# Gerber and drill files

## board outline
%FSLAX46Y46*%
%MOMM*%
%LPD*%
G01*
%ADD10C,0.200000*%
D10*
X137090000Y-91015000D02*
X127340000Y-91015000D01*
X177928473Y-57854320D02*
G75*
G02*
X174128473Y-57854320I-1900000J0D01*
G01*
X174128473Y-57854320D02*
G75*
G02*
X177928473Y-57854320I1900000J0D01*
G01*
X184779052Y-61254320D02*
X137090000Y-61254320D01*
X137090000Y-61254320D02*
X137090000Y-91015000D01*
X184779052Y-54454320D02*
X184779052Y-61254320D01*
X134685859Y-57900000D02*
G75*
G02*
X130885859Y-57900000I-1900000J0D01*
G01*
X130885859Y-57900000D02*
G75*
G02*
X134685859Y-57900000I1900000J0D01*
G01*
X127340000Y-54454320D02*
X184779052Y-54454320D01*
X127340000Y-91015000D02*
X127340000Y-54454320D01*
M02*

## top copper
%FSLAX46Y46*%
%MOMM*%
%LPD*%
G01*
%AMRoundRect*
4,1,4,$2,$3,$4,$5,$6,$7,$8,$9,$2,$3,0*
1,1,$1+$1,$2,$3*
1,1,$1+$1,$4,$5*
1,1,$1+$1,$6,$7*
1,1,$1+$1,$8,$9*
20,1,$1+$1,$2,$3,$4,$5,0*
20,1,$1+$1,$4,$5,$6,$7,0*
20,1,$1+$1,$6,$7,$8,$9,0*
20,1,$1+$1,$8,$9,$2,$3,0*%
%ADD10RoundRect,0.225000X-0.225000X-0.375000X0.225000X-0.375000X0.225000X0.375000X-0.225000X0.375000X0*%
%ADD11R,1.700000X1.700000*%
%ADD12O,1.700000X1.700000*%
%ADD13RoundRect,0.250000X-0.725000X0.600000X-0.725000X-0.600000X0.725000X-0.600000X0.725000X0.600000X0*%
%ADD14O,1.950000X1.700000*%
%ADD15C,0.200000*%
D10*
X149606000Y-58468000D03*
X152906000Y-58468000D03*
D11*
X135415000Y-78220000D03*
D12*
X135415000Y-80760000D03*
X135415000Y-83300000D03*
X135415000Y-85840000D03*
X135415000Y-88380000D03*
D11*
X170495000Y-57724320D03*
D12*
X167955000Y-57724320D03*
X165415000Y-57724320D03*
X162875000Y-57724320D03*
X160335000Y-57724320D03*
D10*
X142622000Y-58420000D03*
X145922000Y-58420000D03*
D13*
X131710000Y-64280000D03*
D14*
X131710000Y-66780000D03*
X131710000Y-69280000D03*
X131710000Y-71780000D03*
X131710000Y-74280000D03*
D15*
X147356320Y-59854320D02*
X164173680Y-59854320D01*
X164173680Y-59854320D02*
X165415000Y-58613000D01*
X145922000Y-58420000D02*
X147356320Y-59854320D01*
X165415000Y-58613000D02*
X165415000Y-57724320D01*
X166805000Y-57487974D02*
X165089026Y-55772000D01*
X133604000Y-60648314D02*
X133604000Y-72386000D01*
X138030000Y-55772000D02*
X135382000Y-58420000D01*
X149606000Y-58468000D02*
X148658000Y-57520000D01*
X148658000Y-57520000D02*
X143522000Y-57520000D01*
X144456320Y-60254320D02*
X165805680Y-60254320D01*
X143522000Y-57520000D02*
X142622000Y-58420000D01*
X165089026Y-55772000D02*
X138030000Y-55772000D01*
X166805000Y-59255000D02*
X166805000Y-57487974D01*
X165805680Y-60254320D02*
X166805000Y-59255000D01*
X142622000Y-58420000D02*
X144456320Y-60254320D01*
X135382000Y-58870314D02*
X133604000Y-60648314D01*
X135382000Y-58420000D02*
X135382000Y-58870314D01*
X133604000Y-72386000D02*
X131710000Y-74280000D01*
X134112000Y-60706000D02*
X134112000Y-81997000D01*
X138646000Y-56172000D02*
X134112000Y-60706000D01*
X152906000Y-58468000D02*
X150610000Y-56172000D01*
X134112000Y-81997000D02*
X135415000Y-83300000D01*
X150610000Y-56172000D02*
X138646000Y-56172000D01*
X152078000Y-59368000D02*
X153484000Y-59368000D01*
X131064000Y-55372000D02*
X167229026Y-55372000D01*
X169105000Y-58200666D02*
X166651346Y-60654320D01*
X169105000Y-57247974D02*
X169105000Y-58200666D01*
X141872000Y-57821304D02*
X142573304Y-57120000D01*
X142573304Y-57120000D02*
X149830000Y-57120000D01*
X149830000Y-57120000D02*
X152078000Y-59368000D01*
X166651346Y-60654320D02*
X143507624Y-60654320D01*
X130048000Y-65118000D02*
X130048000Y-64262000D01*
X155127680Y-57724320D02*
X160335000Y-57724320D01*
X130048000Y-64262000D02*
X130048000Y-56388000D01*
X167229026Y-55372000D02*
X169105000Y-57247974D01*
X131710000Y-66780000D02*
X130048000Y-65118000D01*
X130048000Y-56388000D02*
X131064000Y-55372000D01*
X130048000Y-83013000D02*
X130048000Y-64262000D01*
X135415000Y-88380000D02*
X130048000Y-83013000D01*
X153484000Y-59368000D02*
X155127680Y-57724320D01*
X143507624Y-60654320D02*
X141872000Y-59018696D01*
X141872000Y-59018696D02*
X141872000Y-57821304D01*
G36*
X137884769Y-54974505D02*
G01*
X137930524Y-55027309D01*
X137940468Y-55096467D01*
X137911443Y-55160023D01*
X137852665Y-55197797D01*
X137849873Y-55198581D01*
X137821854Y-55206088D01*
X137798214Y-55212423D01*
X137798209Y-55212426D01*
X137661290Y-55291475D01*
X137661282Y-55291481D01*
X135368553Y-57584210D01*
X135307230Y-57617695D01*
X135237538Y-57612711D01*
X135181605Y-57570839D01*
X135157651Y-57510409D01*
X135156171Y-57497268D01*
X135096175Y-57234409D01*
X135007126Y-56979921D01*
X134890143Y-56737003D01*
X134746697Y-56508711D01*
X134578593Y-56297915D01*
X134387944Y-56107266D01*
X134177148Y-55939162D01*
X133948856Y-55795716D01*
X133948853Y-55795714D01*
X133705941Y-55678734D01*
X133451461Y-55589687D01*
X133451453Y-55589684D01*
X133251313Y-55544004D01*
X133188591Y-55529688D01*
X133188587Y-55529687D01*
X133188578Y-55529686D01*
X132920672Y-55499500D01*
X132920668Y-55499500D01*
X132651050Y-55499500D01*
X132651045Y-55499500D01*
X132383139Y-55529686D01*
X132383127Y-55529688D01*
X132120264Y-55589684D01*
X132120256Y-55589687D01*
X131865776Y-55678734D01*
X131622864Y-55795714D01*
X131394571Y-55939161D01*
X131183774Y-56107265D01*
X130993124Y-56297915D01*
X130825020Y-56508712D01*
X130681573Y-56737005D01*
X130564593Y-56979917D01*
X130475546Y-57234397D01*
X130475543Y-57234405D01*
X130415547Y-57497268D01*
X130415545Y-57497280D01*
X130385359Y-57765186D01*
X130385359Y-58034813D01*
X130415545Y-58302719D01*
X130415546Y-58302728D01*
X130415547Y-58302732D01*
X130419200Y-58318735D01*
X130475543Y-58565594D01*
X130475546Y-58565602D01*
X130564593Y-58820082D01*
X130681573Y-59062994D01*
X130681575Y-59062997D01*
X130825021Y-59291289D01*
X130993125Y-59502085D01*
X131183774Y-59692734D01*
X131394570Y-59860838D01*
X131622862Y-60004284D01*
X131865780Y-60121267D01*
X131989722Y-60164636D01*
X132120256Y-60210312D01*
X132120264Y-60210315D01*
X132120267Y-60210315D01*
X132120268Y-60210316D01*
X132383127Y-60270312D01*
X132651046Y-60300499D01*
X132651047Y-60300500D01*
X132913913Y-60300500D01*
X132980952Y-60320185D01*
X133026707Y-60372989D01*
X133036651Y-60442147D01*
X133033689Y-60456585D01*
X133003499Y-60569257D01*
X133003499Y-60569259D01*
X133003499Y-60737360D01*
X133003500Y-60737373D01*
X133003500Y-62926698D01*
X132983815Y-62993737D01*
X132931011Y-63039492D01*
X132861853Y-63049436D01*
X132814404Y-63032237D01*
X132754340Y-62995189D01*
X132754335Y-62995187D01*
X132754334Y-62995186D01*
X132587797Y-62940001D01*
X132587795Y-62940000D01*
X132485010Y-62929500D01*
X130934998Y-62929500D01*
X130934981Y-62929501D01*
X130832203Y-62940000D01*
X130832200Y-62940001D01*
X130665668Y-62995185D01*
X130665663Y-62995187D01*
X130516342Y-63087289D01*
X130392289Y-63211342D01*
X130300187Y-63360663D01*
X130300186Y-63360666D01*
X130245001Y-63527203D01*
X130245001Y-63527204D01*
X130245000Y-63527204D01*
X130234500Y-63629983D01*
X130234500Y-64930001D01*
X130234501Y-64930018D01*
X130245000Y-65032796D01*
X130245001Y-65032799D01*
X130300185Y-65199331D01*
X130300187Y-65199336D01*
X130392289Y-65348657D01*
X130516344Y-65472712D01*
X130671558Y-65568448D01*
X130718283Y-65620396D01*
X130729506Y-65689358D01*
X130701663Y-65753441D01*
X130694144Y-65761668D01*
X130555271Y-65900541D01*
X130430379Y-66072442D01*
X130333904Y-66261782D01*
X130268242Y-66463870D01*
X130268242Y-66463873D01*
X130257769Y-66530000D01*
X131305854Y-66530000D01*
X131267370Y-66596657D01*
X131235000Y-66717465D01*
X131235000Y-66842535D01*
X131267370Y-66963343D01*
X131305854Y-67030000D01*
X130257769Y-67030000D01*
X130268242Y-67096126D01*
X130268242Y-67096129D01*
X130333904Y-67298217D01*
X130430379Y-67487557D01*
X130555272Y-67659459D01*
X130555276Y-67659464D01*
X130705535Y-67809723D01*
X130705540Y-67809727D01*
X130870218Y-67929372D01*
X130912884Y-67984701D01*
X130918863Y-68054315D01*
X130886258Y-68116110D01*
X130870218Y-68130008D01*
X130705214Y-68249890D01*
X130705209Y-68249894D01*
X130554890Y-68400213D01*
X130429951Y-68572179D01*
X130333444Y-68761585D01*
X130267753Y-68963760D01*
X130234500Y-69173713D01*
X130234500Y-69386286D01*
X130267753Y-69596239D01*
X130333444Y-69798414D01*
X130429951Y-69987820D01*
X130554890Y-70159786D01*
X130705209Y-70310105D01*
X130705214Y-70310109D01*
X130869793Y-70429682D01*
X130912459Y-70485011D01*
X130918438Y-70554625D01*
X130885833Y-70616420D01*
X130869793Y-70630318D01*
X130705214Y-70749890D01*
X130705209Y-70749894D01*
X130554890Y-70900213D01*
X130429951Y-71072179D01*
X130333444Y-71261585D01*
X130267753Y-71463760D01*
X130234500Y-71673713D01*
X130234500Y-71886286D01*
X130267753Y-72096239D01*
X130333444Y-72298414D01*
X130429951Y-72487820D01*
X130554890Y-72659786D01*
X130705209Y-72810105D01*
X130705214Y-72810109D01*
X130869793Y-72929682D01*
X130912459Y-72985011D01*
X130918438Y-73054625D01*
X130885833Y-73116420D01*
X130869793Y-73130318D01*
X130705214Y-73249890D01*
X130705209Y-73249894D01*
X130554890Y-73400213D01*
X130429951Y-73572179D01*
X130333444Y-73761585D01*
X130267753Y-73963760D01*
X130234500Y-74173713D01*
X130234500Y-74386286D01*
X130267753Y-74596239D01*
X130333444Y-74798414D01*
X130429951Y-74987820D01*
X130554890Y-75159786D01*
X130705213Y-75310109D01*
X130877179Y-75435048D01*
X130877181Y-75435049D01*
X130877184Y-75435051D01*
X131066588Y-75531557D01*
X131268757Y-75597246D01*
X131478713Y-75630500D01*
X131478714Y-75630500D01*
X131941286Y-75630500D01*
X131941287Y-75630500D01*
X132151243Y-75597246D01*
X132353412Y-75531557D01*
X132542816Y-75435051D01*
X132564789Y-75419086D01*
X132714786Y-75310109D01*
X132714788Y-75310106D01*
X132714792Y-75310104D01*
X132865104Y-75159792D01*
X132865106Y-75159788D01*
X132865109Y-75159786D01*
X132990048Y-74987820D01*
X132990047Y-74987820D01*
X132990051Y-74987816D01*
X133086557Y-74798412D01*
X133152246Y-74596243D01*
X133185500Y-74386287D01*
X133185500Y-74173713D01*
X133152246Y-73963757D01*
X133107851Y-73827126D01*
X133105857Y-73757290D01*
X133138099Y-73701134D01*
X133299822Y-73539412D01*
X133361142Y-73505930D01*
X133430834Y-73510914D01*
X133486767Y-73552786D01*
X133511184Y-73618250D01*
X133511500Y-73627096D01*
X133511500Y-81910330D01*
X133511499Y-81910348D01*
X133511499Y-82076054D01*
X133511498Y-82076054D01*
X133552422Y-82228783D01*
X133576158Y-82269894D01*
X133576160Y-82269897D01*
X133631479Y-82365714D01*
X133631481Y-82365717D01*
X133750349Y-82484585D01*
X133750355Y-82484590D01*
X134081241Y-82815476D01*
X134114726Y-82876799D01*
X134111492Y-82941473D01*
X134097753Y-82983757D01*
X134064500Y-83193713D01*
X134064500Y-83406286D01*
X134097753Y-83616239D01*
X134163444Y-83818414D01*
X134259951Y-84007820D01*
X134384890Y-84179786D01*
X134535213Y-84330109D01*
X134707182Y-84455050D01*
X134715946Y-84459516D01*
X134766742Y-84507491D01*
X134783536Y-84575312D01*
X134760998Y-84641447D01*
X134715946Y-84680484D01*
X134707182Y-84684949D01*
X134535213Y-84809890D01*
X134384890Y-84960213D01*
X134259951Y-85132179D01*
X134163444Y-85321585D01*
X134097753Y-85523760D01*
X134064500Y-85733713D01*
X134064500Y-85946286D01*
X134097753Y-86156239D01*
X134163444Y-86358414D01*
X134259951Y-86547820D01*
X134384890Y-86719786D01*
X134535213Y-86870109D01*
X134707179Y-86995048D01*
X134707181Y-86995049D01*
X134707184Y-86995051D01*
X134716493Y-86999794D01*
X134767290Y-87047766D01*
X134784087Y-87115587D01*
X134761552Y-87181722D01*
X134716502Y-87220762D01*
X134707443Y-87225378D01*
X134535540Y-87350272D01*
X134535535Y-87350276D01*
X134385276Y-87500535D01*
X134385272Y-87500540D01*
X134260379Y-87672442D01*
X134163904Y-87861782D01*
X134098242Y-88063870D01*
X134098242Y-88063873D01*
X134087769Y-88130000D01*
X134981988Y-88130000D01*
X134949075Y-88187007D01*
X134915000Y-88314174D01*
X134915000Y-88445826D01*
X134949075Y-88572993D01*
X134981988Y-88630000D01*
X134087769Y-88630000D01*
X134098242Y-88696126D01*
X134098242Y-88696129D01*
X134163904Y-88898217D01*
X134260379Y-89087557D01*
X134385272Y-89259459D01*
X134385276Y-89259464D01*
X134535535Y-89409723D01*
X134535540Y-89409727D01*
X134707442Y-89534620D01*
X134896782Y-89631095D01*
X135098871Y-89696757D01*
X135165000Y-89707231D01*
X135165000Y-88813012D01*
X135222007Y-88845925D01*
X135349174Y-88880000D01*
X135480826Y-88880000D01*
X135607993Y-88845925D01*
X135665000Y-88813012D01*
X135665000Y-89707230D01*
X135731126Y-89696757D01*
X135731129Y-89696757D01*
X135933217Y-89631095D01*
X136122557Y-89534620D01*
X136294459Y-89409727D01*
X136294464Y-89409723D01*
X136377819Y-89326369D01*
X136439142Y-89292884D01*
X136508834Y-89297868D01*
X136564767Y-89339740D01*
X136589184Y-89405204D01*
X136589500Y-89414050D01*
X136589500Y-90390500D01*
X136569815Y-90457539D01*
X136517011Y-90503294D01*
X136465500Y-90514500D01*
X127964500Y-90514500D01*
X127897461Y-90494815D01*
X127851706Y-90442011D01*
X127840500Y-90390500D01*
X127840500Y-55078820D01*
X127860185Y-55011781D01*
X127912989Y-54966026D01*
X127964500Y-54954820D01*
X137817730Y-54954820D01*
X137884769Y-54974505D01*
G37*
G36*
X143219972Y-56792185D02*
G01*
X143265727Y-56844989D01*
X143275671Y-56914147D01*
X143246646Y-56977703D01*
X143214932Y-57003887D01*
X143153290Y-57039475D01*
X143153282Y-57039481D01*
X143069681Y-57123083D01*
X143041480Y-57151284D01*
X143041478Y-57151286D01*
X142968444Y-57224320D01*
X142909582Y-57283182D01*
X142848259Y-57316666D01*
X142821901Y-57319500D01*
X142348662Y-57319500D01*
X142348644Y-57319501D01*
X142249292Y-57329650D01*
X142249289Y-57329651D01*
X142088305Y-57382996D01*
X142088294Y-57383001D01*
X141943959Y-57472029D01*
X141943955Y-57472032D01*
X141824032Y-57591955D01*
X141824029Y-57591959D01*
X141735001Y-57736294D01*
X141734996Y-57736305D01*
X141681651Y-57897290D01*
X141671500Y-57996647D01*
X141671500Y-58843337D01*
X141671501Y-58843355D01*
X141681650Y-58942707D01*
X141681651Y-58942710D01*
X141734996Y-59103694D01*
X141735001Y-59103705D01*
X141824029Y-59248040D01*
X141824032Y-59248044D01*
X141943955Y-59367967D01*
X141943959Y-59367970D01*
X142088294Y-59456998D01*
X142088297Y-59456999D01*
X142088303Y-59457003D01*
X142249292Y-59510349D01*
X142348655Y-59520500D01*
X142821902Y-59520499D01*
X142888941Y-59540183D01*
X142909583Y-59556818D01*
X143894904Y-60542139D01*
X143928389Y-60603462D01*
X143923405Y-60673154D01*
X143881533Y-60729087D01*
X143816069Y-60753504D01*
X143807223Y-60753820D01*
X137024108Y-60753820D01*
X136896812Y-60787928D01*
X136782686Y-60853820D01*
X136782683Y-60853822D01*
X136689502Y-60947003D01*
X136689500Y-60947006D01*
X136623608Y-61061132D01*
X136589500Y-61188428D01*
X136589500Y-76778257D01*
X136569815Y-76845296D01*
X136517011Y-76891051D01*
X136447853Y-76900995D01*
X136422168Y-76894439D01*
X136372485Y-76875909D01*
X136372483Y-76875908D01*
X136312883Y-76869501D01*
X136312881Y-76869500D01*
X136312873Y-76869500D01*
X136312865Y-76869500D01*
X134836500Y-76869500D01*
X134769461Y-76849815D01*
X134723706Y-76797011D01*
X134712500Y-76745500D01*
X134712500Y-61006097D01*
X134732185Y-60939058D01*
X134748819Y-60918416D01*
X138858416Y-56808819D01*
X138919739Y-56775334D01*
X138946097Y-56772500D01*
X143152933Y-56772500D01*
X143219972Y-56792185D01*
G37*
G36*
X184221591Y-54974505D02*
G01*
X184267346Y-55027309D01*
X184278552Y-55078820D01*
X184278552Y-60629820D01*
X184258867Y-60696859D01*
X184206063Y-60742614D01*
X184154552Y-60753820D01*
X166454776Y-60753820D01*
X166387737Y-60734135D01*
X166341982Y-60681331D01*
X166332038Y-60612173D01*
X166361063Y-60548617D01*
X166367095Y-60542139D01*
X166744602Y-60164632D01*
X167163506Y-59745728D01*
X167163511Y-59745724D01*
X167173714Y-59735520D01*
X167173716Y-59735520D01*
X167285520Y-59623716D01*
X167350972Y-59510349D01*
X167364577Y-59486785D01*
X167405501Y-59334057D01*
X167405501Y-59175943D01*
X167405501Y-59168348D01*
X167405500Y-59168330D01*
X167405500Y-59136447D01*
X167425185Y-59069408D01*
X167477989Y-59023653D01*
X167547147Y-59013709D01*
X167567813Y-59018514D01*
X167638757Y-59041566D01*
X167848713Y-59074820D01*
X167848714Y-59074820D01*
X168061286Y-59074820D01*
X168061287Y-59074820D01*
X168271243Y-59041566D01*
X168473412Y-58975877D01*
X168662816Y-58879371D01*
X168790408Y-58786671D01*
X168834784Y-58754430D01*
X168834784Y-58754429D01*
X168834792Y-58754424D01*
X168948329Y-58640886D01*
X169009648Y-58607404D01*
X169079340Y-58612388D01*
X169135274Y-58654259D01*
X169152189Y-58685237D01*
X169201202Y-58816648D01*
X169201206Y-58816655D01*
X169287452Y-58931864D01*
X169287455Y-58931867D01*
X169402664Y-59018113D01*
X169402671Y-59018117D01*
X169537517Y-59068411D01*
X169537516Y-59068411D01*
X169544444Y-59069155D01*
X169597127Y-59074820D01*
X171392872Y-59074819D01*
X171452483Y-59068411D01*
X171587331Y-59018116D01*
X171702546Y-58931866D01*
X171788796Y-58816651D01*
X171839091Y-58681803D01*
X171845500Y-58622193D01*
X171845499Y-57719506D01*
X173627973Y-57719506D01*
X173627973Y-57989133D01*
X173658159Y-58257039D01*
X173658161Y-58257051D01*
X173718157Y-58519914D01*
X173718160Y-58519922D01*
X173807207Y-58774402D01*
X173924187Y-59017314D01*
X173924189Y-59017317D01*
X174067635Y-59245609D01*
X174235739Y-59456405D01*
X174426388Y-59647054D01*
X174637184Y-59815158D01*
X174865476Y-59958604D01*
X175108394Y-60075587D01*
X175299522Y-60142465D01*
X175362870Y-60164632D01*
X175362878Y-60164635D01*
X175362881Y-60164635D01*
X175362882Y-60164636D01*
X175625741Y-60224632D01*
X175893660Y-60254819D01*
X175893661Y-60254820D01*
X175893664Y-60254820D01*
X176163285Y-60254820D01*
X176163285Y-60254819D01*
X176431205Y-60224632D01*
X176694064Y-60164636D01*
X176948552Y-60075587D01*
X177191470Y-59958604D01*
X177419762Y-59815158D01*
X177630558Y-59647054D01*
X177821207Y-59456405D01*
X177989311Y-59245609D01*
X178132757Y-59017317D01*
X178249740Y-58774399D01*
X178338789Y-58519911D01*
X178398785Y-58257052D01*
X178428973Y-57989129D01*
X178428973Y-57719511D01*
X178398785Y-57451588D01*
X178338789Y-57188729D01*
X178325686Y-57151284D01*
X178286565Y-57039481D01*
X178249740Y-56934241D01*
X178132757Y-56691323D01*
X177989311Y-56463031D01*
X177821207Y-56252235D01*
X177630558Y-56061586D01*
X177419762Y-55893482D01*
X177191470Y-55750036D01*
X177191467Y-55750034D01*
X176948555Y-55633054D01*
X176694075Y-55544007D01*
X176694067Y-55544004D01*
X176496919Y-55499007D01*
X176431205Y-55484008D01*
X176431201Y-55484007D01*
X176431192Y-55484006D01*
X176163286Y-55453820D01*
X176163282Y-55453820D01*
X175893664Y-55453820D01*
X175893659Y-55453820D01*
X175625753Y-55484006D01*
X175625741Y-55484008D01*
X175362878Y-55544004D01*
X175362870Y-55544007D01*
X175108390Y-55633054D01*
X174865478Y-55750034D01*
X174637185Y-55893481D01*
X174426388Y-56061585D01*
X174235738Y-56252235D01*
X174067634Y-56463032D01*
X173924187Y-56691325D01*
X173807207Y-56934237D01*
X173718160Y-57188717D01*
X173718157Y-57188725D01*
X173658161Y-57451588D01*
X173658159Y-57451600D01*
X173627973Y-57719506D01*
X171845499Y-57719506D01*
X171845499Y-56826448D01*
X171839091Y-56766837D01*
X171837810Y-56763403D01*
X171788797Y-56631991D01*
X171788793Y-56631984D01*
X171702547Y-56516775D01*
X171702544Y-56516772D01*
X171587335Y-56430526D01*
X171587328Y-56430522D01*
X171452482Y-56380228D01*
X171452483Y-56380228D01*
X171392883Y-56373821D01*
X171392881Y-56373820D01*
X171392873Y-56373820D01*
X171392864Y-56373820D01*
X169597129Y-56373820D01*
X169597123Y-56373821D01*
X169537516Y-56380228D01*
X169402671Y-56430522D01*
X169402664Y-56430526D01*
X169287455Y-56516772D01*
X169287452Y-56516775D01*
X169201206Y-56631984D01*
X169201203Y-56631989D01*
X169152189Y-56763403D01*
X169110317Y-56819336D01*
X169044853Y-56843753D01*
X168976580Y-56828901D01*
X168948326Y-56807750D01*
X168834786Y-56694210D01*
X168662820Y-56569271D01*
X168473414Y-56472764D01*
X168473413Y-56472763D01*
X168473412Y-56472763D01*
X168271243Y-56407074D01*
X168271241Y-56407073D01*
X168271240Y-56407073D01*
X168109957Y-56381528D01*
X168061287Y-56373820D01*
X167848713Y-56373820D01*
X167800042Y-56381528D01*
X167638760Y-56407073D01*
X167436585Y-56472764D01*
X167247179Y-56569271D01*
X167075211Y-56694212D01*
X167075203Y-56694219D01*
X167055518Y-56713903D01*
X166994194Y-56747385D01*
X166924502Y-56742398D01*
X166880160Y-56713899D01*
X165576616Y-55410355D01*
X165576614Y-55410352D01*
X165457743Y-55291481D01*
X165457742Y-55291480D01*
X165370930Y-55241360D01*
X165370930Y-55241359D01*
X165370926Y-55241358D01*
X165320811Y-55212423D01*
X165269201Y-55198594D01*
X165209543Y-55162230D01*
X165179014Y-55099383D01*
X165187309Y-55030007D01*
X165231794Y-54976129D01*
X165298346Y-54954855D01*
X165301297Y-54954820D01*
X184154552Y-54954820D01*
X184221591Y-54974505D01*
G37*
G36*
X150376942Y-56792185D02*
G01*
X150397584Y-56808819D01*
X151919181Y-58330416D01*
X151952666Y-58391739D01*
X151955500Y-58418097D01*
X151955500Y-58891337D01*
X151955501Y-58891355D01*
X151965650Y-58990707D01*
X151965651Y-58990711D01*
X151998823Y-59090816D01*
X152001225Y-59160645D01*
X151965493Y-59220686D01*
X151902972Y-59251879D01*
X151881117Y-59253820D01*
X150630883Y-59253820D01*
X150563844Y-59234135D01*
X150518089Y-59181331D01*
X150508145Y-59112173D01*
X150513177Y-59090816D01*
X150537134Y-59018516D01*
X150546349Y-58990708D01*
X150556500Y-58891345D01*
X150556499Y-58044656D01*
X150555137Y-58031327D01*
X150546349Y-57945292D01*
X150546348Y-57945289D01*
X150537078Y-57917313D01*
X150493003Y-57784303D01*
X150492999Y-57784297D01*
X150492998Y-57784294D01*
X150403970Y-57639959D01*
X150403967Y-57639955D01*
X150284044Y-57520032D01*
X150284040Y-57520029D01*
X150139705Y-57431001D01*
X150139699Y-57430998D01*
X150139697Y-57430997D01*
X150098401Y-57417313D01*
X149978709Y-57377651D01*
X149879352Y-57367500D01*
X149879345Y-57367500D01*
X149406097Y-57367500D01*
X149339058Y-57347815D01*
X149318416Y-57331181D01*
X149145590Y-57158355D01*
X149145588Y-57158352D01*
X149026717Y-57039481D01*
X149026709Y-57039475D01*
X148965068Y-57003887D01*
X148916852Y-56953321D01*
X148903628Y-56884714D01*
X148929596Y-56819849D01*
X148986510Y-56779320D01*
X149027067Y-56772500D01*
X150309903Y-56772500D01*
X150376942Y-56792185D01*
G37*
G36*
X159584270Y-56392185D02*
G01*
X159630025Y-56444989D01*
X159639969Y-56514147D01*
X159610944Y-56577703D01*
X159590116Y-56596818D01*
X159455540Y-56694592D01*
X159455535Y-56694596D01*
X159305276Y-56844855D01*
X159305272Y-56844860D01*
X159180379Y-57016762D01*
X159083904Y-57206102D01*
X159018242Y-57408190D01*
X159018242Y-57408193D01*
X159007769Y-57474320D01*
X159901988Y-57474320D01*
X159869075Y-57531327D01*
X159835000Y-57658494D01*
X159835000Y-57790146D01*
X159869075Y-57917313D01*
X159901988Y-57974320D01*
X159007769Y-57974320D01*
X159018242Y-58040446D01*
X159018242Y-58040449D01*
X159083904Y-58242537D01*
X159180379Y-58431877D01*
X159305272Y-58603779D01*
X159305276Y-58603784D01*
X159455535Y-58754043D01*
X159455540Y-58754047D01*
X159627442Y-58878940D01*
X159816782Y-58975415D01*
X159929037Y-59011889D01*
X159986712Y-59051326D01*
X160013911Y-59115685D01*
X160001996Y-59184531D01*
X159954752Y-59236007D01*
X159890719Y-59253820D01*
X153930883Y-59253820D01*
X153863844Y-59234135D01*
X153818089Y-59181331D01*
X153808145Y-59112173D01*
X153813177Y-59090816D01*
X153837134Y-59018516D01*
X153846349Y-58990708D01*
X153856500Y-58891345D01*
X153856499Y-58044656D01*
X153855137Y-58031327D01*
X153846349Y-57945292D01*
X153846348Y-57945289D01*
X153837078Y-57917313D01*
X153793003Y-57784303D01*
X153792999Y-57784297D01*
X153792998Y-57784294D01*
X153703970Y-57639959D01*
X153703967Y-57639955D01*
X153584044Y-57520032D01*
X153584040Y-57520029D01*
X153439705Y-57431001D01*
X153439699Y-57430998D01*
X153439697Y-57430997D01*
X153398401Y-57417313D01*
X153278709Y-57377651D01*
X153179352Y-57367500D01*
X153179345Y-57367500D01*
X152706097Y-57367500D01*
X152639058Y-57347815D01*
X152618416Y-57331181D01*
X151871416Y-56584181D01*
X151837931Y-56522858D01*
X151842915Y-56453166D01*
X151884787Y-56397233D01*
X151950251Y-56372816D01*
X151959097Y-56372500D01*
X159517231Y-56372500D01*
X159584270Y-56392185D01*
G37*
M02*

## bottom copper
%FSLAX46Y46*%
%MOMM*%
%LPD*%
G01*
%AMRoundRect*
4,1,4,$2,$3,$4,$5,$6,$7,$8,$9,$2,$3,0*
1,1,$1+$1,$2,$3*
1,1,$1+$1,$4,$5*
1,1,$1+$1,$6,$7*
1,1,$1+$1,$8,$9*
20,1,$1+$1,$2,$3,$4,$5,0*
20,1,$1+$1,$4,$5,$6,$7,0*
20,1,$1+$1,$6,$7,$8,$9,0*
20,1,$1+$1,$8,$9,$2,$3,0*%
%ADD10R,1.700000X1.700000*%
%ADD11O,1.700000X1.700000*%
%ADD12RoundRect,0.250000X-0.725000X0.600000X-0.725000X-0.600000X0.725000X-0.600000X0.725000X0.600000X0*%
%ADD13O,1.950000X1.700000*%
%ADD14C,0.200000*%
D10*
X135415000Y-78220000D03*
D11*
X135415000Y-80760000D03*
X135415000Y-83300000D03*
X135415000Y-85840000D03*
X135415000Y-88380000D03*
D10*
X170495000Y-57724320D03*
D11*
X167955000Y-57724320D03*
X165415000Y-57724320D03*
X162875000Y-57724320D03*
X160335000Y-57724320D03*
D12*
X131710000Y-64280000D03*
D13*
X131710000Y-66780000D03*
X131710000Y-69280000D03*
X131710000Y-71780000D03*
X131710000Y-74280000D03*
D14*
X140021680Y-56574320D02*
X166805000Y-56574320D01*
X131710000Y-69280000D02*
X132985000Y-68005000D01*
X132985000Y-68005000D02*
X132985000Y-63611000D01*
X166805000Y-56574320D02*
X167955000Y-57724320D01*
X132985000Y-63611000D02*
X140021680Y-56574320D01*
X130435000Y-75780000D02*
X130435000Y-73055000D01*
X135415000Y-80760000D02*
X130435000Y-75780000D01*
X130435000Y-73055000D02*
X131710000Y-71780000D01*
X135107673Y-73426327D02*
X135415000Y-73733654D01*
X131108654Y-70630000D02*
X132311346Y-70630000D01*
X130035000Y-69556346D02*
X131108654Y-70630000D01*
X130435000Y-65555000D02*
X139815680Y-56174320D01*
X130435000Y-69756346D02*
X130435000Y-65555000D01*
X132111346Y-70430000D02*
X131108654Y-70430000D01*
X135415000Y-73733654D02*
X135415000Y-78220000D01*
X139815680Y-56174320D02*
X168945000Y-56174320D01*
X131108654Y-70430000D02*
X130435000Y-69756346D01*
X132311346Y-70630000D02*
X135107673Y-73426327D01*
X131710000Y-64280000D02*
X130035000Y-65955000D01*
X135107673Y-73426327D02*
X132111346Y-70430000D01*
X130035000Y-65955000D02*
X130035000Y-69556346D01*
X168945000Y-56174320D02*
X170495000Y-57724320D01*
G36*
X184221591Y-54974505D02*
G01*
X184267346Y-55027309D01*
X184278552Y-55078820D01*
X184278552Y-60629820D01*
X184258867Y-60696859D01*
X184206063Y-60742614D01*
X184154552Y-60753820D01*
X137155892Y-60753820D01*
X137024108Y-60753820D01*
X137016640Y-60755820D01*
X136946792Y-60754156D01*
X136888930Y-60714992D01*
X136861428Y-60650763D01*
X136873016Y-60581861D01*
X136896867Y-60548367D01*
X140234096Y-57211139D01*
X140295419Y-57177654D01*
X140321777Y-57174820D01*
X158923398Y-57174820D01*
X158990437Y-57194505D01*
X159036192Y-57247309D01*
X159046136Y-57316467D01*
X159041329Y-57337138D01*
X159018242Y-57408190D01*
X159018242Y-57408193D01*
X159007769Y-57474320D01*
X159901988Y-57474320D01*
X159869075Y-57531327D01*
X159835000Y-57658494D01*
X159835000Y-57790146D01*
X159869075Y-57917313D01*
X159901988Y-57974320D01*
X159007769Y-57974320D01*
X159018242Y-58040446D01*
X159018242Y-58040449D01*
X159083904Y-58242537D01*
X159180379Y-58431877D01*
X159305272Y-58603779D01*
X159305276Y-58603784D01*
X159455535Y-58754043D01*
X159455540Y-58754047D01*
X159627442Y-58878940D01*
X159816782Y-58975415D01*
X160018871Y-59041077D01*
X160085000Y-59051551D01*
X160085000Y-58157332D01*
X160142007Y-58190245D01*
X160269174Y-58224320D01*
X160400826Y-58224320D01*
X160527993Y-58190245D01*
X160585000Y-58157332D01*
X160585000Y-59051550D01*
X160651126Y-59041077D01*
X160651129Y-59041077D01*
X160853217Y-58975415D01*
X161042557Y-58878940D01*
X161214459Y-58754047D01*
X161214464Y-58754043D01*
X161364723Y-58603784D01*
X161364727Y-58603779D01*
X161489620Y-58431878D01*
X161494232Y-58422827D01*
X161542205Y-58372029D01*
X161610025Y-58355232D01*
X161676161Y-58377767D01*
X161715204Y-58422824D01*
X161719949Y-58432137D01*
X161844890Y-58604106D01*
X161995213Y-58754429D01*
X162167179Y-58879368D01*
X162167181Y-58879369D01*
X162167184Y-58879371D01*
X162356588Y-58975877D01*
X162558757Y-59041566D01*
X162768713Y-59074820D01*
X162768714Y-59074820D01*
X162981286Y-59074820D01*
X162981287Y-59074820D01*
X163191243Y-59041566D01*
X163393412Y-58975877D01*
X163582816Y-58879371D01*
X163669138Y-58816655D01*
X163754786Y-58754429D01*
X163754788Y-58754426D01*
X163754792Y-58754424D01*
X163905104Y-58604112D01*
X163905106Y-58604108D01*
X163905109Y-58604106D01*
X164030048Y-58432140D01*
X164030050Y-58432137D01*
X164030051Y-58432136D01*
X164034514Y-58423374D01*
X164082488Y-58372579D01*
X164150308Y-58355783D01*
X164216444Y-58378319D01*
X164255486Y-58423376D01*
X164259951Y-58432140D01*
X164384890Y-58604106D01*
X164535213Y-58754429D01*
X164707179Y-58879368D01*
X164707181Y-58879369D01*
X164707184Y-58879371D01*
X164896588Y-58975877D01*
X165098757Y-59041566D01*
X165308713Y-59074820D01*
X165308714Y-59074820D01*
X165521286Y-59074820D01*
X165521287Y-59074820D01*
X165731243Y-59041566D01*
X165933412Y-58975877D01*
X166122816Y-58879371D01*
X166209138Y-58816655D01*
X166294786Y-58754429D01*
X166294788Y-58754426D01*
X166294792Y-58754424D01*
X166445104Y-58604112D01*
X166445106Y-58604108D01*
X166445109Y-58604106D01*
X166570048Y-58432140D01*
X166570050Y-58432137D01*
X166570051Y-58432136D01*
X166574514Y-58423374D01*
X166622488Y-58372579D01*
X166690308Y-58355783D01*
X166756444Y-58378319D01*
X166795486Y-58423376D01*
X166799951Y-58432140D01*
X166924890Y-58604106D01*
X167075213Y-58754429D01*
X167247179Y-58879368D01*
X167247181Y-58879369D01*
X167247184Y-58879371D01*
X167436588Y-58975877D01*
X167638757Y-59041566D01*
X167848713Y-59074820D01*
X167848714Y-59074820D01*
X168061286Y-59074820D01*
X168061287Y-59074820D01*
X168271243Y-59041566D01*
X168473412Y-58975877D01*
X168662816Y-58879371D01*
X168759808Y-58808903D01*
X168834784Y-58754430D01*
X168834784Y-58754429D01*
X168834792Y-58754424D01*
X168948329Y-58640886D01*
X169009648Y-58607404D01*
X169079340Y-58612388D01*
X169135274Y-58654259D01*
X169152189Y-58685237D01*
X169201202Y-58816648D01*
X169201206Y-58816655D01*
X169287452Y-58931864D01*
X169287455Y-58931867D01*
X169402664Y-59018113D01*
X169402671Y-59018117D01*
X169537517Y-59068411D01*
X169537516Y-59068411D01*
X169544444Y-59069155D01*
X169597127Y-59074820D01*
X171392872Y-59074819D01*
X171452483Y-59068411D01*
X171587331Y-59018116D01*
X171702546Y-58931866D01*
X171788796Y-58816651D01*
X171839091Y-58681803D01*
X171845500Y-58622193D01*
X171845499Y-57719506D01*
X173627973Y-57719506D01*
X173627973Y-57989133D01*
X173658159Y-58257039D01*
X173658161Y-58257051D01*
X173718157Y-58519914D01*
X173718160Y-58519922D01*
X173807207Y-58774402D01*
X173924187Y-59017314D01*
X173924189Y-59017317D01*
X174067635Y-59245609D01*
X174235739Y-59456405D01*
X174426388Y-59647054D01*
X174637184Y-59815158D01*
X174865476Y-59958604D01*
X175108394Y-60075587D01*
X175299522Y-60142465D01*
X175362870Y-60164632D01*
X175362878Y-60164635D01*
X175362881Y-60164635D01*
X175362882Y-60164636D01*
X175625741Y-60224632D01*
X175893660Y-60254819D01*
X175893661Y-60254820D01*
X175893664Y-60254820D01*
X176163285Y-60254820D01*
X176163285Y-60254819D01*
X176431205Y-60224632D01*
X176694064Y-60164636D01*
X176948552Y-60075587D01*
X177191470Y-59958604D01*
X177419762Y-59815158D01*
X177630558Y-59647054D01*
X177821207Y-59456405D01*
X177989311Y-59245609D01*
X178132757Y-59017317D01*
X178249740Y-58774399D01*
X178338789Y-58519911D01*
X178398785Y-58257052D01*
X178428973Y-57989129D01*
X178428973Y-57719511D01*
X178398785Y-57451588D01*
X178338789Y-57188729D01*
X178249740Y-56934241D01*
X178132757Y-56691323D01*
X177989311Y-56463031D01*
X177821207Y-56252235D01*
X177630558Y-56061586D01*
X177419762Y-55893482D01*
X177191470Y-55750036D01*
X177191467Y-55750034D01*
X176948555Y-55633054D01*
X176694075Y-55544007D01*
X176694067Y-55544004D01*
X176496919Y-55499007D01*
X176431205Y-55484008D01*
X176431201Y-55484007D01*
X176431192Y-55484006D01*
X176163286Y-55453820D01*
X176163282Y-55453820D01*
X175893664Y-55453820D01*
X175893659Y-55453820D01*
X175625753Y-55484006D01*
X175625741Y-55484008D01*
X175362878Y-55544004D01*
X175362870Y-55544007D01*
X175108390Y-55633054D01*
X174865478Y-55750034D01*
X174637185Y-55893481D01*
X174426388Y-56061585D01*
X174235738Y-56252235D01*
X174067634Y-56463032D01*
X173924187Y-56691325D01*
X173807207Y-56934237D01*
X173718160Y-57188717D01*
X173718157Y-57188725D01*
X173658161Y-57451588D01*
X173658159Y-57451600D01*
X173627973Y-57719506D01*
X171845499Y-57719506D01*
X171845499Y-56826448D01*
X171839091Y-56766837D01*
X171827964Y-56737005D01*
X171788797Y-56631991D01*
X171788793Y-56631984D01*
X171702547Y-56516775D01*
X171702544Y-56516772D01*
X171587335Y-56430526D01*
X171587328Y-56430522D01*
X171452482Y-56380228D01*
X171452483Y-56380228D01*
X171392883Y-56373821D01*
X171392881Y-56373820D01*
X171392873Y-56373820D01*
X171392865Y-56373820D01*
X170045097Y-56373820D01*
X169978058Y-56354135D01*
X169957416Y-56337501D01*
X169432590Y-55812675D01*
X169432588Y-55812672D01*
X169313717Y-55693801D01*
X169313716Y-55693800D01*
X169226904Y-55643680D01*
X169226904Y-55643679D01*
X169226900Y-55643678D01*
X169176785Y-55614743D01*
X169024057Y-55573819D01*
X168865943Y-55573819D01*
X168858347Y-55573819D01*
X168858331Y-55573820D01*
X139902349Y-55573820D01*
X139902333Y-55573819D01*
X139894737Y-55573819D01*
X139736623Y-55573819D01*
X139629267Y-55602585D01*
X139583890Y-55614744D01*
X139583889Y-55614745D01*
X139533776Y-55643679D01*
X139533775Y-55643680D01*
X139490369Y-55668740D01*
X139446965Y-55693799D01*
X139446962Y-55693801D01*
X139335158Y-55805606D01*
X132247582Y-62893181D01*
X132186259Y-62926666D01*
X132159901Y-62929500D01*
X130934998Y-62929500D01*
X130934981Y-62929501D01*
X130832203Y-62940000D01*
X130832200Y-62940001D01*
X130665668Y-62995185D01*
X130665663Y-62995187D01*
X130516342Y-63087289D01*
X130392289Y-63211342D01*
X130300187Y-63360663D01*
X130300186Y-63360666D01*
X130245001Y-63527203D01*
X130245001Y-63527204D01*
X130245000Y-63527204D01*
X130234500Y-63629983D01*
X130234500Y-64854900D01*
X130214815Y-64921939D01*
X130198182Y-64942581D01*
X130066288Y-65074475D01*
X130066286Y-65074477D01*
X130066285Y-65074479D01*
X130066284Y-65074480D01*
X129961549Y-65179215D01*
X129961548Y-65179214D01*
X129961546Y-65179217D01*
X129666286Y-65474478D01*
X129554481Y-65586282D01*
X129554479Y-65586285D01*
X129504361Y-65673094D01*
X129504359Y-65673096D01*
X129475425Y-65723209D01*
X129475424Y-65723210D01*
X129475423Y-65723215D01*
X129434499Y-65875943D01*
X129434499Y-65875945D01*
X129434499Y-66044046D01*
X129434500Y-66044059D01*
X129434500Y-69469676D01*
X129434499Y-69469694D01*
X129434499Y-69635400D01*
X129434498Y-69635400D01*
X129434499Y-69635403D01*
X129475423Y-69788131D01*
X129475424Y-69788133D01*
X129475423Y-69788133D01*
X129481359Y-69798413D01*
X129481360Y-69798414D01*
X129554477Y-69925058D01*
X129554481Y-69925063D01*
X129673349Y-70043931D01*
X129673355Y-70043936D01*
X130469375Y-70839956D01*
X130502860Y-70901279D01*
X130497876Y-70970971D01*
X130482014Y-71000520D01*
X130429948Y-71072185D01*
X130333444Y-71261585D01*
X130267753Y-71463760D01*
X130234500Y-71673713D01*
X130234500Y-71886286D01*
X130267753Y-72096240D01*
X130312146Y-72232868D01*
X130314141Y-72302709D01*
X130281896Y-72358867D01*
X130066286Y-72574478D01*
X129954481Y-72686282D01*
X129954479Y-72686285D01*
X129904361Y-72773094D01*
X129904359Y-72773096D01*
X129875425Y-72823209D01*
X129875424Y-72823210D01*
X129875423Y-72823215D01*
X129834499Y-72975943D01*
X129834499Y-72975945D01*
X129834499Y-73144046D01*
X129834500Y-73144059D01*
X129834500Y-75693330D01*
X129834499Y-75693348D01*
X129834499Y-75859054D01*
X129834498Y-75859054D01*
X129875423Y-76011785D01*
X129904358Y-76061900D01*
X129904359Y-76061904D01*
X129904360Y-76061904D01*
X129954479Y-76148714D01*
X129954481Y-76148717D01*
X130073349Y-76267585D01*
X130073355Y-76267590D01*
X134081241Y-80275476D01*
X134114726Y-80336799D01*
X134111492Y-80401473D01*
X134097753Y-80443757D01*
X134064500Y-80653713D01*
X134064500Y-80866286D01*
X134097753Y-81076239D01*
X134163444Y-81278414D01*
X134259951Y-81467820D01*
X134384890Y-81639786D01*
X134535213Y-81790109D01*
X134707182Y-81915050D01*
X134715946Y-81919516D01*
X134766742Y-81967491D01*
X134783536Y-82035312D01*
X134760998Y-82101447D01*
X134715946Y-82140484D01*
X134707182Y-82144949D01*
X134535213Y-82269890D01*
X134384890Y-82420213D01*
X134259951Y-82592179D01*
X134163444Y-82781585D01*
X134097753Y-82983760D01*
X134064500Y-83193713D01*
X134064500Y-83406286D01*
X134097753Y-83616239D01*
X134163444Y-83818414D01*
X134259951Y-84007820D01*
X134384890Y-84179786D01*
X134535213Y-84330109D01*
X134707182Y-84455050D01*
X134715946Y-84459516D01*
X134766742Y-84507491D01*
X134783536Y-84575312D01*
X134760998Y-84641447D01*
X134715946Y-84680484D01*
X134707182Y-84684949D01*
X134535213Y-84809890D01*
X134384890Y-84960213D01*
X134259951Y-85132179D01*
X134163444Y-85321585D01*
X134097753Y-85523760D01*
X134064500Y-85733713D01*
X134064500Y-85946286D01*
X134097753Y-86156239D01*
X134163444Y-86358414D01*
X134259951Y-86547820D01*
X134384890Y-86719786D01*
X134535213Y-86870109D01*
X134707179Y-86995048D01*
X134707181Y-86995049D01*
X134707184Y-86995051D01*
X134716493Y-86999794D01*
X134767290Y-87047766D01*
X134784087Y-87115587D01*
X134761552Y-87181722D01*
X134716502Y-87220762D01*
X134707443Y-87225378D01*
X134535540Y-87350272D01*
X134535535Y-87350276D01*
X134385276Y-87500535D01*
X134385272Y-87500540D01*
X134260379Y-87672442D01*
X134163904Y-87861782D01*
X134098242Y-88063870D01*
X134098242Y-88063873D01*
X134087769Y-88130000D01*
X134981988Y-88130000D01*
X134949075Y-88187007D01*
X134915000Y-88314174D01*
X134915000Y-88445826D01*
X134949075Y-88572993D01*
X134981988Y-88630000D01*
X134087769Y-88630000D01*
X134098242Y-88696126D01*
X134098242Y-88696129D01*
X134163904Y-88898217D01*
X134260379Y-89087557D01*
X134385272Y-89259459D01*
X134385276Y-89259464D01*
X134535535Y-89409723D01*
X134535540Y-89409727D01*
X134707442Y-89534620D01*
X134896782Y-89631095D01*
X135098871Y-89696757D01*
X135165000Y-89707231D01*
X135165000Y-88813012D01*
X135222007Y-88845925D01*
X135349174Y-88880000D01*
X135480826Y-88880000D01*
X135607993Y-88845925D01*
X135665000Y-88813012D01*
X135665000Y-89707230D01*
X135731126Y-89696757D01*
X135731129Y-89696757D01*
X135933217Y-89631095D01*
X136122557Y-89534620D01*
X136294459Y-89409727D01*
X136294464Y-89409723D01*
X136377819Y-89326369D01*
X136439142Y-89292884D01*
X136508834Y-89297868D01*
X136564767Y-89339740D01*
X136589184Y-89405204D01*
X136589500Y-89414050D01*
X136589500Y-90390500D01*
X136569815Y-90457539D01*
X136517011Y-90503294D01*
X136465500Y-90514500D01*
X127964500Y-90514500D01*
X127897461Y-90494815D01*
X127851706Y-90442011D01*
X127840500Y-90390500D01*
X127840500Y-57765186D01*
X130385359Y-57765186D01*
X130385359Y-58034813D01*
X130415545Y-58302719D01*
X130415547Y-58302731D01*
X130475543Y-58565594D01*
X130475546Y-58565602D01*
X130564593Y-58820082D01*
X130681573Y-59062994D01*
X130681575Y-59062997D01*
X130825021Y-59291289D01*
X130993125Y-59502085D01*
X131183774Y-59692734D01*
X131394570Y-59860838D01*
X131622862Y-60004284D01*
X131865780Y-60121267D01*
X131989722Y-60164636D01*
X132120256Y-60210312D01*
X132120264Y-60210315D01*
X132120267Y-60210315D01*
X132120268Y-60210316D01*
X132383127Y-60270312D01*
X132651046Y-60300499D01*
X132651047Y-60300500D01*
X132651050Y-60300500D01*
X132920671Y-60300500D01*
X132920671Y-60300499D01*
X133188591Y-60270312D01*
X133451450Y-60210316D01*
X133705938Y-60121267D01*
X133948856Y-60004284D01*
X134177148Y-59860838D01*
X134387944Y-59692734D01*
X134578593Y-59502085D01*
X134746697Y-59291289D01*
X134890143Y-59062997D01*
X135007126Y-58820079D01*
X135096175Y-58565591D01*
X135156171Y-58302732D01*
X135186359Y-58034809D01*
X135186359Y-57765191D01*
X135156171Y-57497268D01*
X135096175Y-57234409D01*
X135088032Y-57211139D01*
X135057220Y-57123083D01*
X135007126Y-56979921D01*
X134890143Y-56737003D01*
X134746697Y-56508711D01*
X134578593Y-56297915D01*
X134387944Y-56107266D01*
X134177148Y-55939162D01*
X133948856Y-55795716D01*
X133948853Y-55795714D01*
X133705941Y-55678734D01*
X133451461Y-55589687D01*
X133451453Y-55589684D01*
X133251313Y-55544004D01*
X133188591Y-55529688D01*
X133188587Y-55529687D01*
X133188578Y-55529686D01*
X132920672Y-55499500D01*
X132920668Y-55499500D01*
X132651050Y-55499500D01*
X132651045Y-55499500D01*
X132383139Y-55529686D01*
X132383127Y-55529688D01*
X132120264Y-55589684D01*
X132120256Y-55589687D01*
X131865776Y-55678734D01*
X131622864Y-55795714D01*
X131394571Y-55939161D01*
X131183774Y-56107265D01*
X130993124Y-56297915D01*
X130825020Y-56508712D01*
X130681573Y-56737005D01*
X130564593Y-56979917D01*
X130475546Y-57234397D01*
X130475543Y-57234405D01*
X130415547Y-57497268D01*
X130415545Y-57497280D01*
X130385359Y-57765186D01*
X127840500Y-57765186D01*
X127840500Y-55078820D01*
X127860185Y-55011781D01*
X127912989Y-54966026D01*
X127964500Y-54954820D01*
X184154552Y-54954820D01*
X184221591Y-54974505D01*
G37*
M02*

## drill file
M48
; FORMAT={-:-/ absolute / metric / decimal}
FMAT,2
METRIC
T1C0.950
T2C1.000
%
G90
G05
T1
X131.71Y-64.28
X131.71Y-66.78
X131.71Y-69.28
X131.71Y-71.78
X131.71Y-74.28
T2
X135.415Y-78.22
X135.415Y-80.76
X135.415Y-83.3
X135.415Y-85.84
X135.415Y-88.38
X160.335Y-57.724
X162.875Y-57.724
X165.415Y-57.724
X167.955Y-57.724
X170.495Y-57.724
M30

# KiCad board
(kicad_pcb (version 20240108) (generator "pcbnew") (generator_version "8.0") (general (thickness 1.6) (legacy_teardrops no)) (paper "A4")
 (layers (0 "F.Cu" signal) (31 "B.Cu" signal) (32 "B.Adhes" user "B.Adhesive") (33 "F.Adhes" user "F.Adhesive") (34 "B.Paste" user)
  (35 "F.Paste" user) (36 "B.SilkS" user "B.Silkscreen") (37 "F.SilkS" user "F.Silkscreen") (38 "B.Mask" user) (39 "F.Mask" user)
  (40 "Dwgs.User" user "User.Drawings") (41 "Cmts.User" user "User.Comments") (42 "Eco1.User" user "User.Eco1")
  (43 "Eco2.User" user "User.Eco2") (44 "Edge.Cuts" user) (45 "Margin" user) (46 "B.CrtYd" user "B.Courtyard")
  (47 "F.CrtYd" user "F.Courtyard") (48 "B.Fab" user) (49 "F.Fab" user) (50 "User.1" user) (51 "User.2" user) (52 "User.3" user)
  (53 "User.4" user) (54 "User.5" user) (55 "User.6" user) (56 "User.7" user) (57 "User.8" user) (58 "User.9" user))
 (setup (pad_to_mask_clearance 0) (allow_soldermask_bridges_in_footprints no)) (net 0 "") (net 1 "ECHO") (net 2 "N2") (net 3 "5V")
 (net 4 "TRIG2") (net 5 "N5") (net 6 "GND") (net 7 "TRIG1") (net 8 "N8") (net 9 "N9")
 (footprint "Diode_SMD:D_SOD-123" (layer "F.Cu") (at 151.256 58.468)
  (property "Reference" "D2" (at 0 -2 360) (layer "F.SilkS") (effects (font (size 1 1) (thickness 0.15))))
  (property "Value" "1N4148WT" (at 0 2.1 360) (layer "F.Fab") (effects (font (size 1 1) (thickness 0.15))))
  (pad "1" smd roundrect (at -1.65 0) (size 0.9 1.2) (layers "F.Cu" "F.Paste" "F.Mask") (roundrect_rratio 0.25) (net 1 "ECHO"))
  (pad "2" smd roundrect (at 1.65 0) (size 0.9 1.2) (layers "F.Cu" "F.Paste" "F.Mask") (roundrect_rratio 0.25) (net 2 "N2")))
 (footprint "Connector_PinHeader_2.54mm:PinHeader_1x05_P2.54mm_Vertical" (layer "F.Cu") (at 135.415 78.22)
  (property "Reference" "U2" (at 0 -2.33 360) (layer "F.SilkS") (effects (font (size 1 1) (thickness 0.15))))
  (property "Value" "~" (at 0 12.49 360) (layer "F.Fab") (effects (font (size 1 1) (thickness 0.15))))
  (pad "1" thru_hole rect (at 0 0) (size 1.7 1.7) (drill 1) (layers "*.Cu" "*.Mask") (remove_unused_layers no) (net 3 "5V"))
  (pad "2" thru_hole oval (at 0 2.54) (size 1.7 1.7) (drill 1) (layers "*.Cu" "*.Mask") (remove_unused_layers no) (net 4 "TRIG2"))
  (pad "3" thru_hole oval (at 0 5.08) (size 1.7 1.7) (drill 1) (layers "*.Cu" "*.Mask") (remove_unused_layers no) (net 2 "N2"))
  (pad "4" thru_hole oval (at 0 7.62) (size 1.7 1.7) (drill 1) (layers "*.Cu" "*.Mask") (remove_unused_layers no) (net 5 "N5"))
  (pad "5" thru_hole oval (at 0 10.16) (size 1.7 1.7) (drill 1) (layers "*.Cu" "*.Mask") (remove_unused_layers no) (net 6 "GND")))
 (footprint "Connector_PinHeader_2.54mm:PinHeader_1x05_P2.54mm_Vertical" (layer "F.Cu") (at 170.495 57.72432 -90)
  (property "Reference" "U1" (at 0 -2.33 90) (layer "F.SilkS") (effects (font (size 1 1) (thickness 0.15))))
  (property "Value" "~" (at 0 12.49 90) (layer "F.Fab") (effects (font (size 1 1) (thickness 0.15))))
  (pad "1" thru_hole rect (at 0 0 270) (size 1.7 1.7) (drill 1) (layers "*.Cu" "*.Mask") (remove_unused_layers no) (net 3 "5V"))
  (pad "2" thru_hole oval (at 0 2.54 270) (size 1.7 1.7) (drill 1) (layers "*.Cu" "*.Mask") (remove_unused_layers no) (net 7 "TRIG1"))
  (pad "3" thru_hole oval (at 0 5.08 270) (size 1.7 1.7) (drill 1) (layers "*.Cu" "*.Mask") (remove_unused_layers no) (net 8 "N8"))
  (pad "4" thru_hole oval (at 0 7.62 270) (size 1.7 1.7) (drill 1) (layers "*.Cu" "*.Mask") (remove_unused_layers no) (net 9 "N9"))
  (pad "5" thru_hole oval (at 0 10.16 270) (size 1.7 1.7) (drill 1) (layers "*.Cu" "*.Mask") (remove_unused_layers no) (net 6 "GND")))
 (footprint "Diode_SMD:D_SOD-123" (layer "F.Cu") (at 144.272 58.42)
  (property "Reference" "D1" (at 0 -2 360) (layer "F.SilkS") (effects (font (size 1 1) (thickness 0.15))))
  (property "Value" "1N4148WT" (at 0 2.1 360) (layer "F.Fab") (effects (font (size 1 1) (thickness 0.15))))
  (pad "1" smd roundrect (at -1.65 0) (size 0.9 1.2) (layers "F.Cu" "F.Paste" "F.Mask") (roundrect_rratio 0.25) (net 1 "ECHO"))
  (pad "2" smd roundrect (at 1.65 0) (size 0.9 1.2) (layers "F.Cu" "F.Paste" "F.Mask") (roundrect_rratio 0.25) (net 8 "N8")))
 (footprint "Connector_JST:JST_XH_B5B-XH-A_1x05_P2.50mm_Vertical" (layer "B.Cu") (at 131.71 64.28 -90)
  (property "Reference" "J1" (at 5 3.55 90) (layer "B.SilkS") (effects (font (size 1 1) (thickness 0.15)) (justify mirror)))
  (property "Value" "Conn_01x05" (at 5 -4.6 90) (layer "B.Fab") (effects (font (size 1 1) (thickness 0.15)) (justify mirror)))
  (pad "1" thru_hole roundrect (at 0 0 270) (size 1.7 1.95) (drill 0.95) (layers "*.Cu" "*.Mask") (remove_unused_layers no)
   (roundrect_rratio 0.147059) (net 3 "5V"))
  (pad "2" thru_hole oval (at 2.5 0 270) (size 1.7 1.95) (drill 0.95) (layers "*.Cu" "*.Mask") (remove_unused_layers no) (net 6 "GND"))
  (pad "3" thru_hole oval (at 5 0 270) (size 1.7 1.95) (drill 0.95) (layers "*.Cu" "*.Mask") (remove_unused_layers no) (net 7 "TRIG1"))
  (pad "4" thru_hole oval (at 7.5 0 270) (size 1.7 1.95) (drill 0.95) (layers "*.Cu" "*.Mask") (remove_unused_layers no) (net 4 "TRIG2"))
  (pad "5" thru_hole oval (at 10 0 270) (size 1.7 1.95) (drill 0.95) (layers "*.Cu" "*.Mask") (remove_unused_layers no) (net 1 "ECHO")))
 (gr_line (start 137.09 91.015) (end 127.34 91.015) (stroke (width 0.2) (type default)) (layer "Edge.Cuts"))
 (gr_circle (center 176.028473 57.85432) (end 174.128473 57.85432) (stroke (width 0.2) (type default)) (fill none) (layer "Edge.Cuts"))
 (gr_line (start 184.779052 61.25432) (end 137.09 61.25432) (stroke (width 0.2) (type default)) (layer "Edge.Cuts"))
 (gr_line (start 137.09 61.25432) (end 137.09 91.015) (stroke (width 0.2) (type default)) (layer "Edge.Cuts"))
 (gr_line (start 184.779052 54.45432) (end 184.779052 61.25432) (stroke (width 0.2) (type default)) (layer "Edge.Cuts"))
 (gr_circle (center 132.785859 57.9) (end 130.885859 57.9) (stroke (width 0.2) (type default)) (fill none) (layer "Edge.Cuts"))
 (gr_line (start 127.34 54.45432) (end 184.779052 54.45432) (stroke (width 0.2) (type default)) (layer "Edge.Cuts"))
 (gr_line (start 127.34 91.015) (end 127.34 54.45432) (stroke (width 0.2) (type default)) (layer "Edge.Cuts"))
 (segment (start 147.35632 59.85432) (end 164.17368 59.85432) (width 0.2) (layer "F.Cu") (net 8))
 (segment (start 164.17368 59.85432) (end 165.415 58.613) (width 0.2) (layer "F.Cu") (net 8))
 (segment (start 145.922 58.42) (end 147.35632 59.85432) (width 0.2) (layer "F.Cu") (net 8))
 (segment (start 165.415 58.613) (end 165.415 57.72432) (width 0.2) (layer "F.Cu") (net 8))
 (segment (start 166.805 57.487974) (end 165.089026 55.772) (width 0.2) (layer "F.Cu") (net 1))
 (segment (start 133.604 60.648314) (end 133.604 72.386) (width 0.2) (layer "F.Cu") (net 1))
 (segment (start 138.03 55.772) (end 135.382 58.42) (width 0.2) (layer "F.Cu") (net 1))
 (segment (start 149.606 58.468) (end 148.658 57.52) (width 0.2) (layer "F.Cu") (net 1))
 (segment (start 148.658 57.52) (end 143.522 57.52) (width 0.2) (layer "F.Cu") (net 1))
 (segment (start 144.45632 60.25432) (end 165.80568 60.25432) (width 0.2) (layer "F.Cu") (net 1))
 (segment (start 143.522 57.52) (end 142.622 58.42) (width 0.2) (layer "F.Cu") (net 1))
 (segment (start 165.089026 55.772) (end 138.03 55.772) (width 0.2) (layer "F.Cu") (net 1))
 (segment (start 166.805 59.255) (end 166.805 57.487974) (width 0.2) (layer "F.Cu") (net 1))
 (segment (start 165.80568 60.25432) (end 166.805 59.255) (width 0.2) (layer "F.Cu") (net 1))
 (segment (start 142.622 58.42) (end 144.45632 60.25432) (width 0.2) (layer "F.Cu") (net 1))
 (segment (start 135.382 58.870314) (end 133.604 60.648314) (width 0.2) (layer "F.Cu") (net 1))
 (segment (start 135.382 58.42) (end 135.382 58.870314) (width 0.2) (layer "F.Cu") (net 1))
 (segment (start 133.604 72.386) (end 131.71 74.28) (width 0.2) (layer "F.Cu") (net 1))
 (segment (start 134.112 60.706) (end 134.112 81.997) (width 0.2) (layer "F.Cu") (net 2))
 (segment (start 138.646 56.172) (end 134.112 60.706) (width 0.2) (layer "F.Cu") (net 2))
 (segment (start 152.906 58.468) (end 150.61 56.172) (width 0.2) (layer "F.Cu") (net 2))
 (segment (start 134.112 81.997) (end 135.415 83.3) (width 0.2) (layer "F.Cu") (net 2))
 (segment (start 150.61 56.172) (end 138.646 56.172) (width 0.2) (layer "F.Cu") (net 2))
 (segment (start 152.078 59.368) (end 153.484 59.368) (width 0.2) (layer "F.Cu") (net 6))
 (segment (start 131.064 55.372) (end 167.229026 55.372) (width 0.2) (layer "F.Cu") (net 6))
 (segment (start 169.105 58.200666) (end 166.651346 60.65432) (width 0.2) (layer "F.Cu") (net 6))
 (segment (start 169.105 57.247974) (end 169.105 58.200666) (width 0.2) (layer "F.Cu") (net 6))
 (segment (start 141.872 57.821304) (end 142.573304 57.12) (width 0.2) (layer "F.Cu") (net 6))
 (segment (start 142.573304 57.12) (end 149.83 57.12) (width 0.2) (layer "F.Cu") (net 6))
 (segment (start 149.83 57.12) (end 152.078 59.368) (width 0.2) (layer "F.Cu") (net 6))
 (segment (start 166.651346 60.65432) (end 143.507624 60.65432) (width 0.2) (layer "F.Cu") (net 6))
 (segment (start 130.048 65.118) (end 130.048 64.262) (width 0.2) (layer "F.Cu") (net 6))
 (segment (start 155.12768 57.72432) (end 160.335 57.72432) (width 0.2) (layer "F.Cu") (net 6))
 (segment (start 130.048 64.262) (end 130.048 56.388) (width 0.2) (layer "F.Cu") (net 6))
 (segment (start 167.229026 55.372) (end 169.105 57.247974) (width 0.2) (layer "F.Cu") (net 6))
 (segment (start 131.71 66.78) (end 130.048 65.118) (width 0.2) (layer "F.Cu") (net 6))
 (segment (start 130.048 56.388) (end 131.064 55.372) (width 0.2) (layer "F.Cu") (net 6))
 (segment (start 130.048 83.013) (end 130.048 64.262) (width 0.2) (layer "F.Cu") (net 6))
 (segment (start 135.415 88.38) (end 130.048 83.013) (width 0.2) (layer "F.Cu") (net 6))
 (segment (start 153.484 59.368) (end 155.12768 57.72432) (width 0.2) (layer "F.Cu") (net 6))
 (segment (start 143.507624 60.65432) (end 141.872 59.018696) (width 0.2) (layer "F.Cu") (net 6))
 (segment (start 141.872 59.018696) (end 141.872 57.821304) (width 0.2) (layer "F.Cu") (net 6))
 (segment (start 140.02168 56.57432) (end 166.805 56.57432) (width 0.2) (layer "B.Cu") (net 7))
 (segment (start 131.71 69.28) (end 132.985 68.005) (width 0.2) (layer "B.Cu") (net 7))
 (segment (start 132.985 68.005) (end 132.985 63.611) (width 0.2) (layer "B.Cu") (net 7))
 (segment (start 166.805 56.57432) (end 167.955 57.72432) (width 0.2) (layer "B.Cu") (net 7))
 (segment (start 132.985 63.611) (end 140.02168 56.57432) (width 0.2) (layer "B.Cu") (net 7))
 (segment (start 130.435 75.78) (end 130.435 73.055) (width 0.2) (layer "B.Cu") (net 4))
 (segment (start 135.415 80.76) (end 130.435 75.78) (width 0.2) (layer "B.Cu") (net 4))
 (segment (start 130.435 73.055) (end 131.71 71.78) (width 0.2) (layer "B.Cu") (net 4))
 (segment (start 135.107673 73.426327) (end 135.415 73.733654) (width 0.2) (layer "B.Cu") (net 3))
 (segment (start 131.108654 70.63) (end 132.311346 70.63) (width 0.2) (layer "B.Cu") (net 3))
 (segment (start 130.035 69.556346) (end 131.108654 70.63) (width 0.2) (layer "B.Cu") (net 3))
 (segment (start 130.435 65.555) (end 139.81568 56.17432) (width 0.2) (layer "B.Cu") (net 3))
 (segment (start 130.435 69.756346) (end 130.435 65.555) (width 0.2) (layer "B.Cu") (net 3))
 (segment (start 132.111346 70.43) (end 131.108654 70.43) (width 0.2) (layer "B.Cu") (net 3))
 (segment (start 135.415 73.733654) (end 135.415 78.22) (width 0.2) (layer "B.Cu") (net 3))
 (segment (start 139.81568 56.17432) (end 168.945 56.17432) (width 0.2) (layer "B.Cu") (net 3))
 (segment (start 131.108654 70.43) (end 130.435 69.756346) (width 0.2) (layer "B.Cu") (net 3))
 (segment (start 132.311346 70.63) (end 135.107673 73.426327) (width 0.2) (layer "B.Cu") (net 3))
 (segment (start 131.71 64.28) (end 130.035 65.955) (width 0.2) (layer "B.Cu") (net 3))
 (segment (start 135.107673 73.426327) (end 132.111346 70.43) (width 0.2) (layer "B.Cu") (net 3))
 (segment (start 130.035 65.955) (end 130.035 69.556346) (width 0.2) (layer "B.Cu") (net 3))
 (segment (start 168.945 56.17432) (end 170.495 57.72432) (width 0.2) (layer "B.Cu") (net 3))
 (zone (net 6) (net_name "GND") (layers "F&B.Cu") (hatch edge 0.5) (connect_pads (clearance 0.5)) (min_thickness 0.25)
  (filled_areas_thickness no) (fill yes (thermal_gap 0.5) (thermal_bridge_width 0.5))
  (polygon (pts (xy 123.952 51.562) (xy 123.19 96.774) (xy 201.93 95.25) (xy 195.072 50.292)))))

